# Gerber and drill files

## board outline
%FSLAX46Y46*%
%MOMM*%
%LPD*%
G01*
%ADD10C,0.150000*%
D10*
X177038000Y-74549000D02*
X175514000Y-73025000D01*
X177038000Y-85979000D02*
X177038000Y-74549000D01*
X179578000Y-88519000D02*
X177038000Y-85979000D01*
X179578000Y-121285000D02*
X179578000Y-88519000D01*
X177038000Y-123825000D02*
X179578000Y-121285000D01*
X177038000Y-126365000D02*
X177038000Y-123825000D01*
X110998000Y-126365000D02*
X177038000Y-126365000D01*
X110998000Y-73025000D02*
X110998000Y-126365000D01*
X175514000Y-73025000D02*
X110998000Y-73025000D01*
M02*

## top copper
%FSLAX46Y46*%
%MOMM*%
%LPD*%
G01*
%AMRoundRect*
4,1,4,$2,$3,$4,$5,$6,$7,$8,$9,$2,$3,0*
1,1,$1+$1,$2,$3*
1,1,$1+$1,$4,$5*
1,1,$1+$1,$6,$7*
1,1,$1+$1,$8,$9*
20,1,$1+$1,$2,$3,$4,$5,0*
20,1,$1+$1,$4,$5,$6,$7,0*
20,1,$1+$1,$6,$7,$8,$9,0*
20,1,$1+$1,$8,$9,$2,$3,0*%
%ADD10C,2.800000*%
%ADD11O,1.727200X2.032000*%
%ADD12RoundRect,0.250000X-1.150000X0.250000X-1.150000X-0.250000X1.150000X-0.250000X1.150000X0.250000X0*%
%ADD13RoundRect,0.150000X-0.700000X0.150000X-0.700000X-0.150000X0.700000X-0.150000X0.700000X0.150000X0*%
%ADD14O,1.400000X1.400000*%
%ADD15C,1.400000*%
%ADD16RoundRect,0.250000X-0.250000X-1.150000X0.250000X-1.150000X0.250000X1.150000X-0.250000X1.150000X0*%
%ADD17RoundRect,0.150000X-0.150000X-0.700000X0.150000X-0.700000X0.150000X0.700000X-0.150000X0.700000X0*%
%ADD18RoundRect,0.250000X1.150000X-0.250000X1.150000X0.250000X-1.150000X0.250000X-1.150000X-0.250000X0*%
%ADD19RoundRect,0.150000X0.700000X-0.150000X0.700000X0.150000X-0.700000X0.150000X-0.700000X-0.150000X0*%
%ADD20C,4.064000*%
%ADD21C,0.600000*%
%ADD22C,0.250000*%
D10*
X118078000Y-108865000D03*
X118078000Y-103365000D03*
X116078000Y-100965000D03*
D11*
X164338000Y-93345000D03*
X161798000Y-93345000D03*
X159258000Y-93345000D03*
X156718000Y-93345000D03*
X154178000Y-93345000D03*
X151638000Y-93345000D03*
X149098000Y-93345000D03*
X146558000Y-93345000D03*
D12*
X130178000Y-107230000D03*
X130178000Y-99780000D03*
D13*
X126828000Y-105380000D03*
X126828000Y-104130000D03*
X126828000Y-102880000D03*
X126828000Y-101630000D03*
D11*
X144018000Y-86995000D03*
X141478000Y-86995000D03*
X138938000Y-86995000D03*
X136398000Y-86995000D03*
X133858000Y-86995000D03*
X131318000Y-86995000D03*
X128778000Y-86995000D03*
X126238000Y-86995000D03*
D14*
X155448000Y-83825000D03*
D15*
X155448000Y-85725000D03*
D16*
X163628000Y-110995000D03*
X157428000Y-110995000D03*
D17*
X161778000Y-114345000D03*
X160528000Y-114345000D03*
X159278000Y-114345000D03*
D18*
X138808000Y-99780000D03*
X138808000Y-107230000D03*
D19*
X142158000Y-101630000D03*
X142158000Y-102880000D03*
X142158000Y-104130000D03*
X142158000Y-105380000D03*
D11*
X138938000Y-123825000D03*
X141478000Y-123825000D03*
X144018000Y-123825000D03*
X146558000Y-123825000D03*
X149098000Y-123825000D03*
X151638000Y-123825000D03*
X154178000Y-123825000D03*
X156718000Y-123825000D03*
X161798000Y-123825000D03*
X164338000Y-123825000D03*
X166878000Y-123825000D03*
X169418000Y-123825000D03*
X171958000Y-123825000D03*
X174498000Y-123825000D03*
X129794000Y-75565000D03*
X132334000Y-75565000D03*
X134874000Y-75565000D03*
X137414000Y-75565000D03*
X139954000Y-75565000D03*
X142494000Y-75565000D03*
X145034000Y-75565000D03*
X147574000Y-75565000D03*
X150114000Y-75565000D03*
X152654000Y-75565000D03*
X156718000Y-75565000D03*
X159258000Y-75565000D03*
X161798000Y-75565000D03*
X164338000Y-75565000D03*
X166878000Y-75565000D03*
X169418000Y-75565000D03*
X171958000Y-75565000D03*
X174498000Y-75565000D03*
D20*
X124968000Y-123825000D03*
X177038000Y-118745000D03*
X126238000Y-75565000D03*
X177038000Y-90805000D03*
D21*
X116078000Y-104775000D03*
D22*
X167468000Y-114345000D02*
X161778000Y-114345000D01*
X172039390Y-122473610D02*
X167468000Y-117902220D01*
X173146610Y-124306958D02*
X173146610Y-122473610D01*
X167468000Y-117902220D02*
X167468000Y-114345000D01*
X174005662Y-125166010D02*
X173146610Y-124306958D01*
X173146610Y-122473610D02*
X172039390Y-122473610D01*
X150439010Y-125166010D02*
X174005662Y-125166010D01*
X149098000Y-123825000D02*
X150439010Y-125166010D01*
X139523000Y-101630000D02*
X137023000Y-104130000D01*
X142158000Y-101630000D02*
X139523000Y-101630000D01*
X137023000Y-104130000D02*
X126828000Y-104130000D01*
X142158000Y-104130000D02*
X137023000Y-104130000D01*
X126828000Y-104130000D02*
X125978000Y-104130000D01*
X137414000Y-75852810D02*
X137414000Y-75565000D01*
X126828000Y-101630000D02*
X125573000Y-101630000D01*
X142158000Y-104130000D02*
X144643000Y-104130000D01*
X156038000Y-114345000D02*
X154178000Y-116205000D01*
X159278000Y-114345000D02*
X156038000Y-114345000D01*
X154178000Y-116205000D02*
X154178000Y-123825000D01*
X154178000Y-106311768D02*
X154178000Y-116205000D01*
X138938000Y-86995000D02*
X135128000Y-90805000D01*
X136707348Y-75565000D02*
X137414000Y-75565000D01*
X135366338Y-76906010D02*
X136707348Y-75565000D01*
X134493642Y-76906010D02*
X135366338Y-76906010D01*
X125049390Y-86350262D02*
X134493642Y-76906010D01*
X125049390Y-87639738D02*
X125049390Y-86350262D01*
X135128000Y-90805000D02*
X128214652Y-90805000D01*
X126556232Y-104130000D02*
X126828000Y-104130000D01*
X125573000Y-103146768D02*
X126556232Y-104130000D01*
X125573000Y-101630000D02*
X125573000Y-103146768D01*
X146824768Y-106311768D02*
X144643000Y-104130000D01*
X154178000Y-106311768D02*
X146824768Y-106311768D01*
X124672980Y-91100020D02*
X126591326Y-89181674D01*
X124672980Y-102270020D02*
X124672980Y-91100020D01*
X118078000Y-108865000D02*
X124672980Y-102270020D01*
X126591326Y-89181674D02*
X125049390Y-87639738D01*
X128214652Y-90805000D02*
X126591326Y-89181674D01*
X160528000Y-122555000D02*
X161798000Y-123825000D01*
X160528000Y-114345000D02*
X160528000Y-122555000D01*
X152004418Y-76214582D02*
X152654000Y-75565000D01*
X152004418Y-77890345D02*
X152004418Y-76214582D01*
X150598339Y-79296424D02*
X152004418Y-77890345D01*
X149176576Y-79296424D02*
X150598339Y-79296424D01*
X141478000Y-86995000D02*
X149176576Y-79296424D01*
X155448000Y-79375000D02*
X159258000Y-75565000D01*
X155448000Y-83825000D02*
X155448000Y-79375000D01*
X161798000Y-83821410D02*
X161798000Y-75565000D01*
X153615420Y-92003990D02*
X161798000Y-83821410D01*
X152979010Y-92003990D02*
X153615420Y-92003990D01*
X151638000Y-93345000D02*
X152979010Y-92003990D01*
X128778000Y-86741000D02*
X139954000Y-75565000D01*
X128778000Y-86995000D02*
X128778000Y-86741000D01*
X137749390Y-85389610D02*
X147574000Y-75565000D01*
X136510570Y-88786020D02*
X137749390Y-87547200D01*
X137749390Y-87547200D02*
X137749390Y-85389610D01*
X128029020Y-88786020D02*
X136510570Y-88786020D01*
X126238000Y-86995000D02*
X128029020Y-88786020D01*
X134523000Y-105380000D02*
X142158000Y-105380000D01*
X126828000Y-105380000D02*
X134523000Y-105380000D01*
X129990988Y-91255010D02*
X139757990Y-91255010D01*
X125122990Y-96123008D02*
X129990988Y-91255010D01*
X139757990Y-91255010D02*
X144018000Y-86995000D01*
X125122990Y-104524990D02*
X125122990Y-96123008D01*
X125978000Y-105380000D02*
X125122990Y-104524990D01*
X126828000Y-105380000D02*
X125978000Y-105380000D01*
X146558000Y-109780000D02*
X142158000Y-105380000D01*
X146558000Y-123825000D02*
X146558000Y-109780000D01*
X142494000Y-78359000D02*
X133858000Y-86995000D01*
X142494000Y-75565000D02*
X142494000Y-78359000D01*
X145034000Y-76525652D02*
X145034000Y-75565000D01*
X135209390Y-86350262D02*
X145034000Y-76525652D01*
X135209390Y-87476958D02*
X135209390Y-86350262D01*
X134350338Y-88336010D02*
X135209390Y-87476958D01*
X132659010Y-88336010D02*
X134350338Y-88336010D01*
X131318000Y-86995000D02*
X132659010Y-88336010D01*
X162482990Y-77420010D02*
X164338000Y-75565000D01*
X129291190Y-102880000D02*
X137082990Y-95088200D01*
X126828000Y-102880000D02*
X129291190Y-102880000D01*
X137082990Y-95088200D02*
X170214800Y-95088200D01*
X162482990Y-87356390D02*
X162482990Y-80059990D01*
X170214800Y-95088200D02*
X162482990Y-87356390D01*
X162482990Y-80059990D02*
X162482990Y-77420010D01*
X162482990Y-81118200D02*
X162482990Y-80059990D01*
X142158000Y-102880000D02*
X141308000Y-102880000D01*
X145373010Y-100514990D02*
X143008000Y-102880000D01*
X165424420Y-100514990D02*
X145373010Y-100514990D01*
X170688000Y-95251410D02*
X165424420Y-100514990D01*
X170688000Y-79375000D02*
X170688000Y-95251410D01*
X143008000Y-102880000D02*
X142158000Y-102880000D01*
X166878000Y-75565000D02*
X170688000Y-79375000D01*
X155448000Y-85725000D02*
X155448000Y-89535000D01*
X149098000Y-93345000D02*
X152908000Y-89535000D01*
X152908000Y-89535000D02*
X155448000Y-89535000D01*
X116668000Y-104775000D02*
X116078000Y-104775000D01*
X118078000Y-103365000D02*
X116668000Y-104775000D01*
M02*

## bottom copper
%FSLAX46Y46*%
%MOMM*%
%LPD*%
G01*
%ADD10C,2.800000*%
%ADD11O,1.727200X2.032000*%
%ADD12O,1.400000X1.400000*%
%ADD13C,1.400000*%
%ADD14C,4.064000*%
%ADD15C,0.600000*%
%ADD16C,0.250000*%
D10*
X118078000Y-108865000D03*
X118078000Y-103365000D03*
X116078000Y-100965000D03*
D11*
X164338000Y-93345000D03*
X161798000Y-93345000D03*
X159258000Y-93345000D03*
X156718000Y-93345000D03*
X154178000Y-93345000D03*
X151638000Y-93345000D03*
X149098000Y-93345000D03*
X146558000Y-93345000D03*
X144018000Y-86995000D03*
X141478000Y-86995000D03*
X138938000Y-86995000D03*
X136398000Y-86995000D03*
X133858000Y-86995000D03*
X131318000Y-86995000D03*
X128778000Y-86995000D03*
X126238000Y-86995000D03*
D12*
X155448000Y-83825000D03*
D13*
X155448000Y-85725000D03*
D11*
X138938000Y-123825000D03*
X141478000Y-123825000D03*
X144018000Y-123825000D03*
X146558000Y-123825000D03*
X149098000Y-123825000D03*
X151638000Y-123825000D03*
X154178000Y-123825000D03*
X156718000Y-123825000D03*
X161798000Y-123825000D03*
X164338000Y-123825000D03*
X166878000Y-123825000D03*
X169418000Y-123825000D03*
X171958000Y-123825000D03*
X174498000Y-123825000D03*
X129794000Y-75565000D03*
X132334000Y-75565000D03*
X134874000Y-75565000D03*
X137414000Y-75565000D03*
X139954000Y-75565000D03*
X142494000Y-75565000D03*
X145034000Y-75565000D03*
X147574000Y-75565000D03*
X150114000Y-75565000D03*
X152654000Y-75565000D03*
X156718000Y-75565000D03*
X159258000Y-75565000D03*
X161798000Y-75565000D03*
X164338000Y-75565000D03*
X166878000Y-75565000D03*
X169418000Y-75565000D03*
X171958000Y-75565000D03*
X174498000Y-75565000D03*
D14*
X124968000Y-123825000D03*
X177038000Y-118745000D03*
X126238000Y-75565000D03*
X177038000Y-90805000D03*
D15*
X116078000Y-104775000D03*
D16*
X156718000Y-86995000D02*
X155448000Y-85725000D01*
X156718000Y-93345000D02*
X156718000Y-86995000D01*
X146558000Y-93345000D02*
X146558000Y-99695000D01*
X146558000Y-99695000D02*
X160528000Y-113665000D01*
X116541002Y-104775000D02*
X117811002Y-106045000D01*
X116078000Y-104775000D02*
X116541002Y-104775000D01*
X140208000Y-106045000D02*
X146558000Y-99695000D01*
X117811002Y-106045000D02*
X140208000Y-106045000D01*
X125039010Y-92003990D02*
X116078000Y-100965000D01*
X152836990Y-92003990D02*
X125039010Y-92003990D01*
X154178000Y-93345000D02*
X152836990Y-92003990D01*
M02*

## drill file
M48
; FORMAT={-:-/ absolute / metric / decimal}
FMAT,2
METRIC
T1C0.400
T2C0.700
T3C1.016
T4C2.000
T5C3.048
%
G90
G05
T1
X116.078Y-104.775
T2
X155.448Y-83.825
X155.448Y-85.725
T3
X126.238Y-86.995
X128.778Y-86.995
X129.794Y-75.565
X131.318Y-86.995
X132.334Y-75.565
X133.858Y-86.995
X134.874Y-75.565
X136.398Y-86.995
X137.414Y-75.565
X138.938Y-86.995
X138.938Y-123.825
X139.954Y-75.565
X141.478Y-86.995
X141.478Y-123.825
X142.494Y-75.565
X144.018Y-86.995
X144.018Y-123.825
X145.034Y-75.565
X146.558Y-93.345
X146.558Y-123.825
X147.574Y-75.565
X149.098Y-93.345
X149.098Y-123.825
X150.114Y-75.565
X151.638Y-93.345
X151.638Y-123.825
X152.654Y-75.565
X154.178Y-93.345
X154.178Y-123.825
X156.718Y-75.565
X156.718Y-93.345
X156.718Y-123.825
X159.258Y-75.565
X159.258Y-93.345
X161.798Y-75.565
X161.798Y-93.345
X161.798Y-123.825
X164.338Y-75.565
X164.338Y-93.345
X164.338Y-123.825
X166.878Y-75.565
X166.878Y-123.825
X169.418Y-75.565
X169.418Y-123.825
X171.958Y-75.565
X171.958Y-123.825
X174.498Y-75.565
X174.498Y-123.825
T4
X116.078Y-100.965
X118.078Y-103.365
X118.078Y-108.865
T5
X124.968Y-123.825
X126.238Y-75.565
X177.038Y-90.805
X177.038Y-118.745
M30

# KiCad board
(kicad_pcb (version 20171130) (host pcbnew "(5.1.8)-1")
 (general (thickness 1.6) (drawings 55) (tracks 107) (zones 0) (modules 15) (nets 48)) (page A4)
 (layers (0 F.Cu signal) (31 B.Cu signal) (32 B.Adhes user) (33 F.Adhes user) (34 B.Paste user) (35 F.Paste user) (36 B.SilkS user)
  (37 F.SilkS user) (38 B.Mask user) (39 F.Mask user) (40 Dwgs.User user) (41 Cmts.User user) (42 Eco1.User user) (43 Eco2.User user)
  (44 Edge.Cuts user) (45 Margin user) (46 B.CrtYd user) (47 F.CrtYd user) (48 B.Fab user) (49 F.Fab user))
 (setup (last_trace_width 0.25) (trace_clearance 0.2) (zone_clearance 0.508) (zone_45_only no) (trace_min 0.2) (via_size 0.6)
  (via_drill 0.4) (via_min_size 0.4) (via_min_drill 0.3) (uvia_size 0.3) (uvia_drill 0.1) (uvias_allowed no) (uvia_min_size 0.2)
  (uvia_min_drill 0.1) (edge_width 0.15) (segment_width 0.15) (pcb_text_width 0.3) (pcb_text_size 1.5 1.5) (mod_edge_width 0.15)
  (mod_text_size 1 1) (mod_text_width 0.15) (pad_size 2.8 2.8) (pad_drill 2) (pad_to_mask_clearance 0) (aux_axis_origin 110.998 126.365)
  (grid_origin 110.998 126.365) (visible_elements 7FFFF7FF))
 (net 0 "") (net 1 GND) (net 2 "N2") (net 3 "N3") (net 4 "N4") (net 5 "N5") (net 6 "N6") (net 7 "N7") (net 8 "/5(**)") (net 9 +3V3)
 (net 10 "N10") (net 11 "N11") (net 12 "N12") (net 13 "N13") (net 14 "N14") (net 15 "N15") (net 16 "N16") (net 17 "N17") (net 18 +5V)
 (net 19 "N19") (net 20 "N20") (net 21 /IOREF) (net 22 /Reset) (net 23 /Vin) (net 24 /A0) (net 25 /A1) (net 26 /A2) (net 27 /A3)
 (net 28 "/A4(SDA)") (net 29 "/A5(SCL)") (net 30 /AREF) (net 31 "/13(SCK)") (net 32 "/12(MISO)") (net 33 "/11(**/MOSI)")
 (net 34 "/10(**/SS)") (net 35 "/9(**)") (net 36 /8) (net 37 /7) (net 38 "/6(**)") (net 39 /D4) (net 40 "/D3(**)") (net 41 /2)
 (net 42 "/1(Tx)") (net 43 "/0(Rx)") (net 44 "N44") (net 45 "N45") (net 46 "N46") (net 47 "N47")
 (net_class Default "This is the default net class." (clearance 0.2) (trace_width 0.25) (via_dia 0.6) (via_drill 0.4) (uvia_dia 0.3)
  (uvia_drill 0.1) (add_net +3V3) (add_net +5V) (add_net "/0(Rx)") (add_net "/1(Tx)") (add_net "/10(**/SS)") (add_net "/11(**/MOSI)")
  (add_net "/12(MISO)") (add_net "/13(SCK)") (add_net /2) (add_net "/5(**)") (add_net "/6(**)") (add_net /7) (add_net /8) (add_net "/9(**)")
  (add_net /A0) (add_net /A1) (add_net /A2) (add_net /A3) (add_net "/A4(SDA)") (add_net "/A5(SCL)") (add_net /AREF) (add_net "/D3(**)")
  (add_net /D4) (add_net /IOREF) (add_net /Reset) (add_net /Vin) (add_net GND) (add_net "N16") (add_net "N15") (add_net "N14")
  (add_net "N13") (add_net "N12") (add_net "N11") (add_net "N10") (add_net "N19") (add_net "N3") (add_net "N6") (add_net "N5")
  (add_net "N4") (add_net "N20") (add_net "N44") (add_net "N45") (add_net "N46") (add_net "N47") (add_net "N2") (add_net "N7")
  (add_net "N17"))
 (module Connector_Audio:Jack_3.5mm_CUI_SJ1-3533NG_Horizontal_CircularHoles (layer F.Cu) (at 116.078 100.965)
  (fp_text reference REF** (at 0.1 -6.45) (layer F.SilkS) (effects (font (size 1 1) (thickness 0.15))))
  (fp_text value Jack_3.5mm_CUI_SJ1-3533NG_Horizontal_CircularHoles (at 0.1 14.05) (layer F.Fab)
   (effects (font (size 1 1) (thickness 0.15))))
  (pad R thru_hole circle (at 2 7.9) (size 2.8 2.8) (drill 2) (layers *.Cu *.Mask) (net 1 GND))
  (pad T thru_hole circle (at 2 2.4) (size 2.8 2.8) (drill 2) (layers *.Cu *.Mask) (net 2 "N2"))
  (pad S thru_hole circle (at 0 0) (size 2.8 2.8) (drill 2) (layers *.Cu *.Mask) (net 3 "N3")))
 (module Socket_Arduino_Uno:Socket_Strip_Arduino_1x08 (layer F.Cu) (at 146.558 93.345)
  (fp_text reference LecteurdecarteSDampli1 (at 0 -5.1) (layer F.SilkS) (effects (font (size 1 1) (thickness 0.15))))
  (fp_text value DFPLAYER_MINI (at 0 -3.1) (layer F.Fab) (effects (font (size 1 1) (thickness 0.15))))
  (pad 8 thru_hole oval (at 17.78 0) (size 1.7272 2.032) (drill 1.016) (layers *.Cu *.Mask F.SilkS) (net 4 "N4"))
  (pad 7 thru_hole oval (at 15.24 0) (size 1.7272 2.032) (drill 1.016) (layers *.Cu *.Mask F.SilkS) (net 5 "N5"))
  (pad 6 thru_hole oval (at 12.7 0) (size 1.7272 2.032) (drill 1.016) (layers *.Cu *.Mask F.SilkS) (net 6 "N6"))
  (pad 5 thru_hole oval (at 10.16 0) (size 1.7272 2.032) (drill 1.016) (layers *.Cu *.Mask F.SilkS) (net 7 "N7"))
  (pad 4 thru_hole oval (at 7.62 0) (size 1.7272 2.032) (drill 1.016) (layers *.Cu *.Mask F.SilkS) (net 3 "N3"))
  (pad 3 thru_hole oval (at 5.08 0) (size 1.7272 2.032) (drill 1.016) (layers *.Cu *.Mask F.SilkS) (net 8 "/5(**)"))
  (pad 2 thru_hole oval (at 2.54 0) (size 1.7272 2.032) (drill 1.016) (layers *.Cu *.Mask F.SilkS) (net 7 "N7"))
  (pad 1 thru_hole oval (at 0 0) (size 1.7272 2.032) (drill 1.016) (layers *.Cu *.Mask F.SilkS) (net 2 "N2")))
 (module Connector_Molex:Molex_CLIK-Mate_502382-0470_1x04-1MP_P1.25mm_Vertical (layer F.Cu) (at 128.778 103.505 270)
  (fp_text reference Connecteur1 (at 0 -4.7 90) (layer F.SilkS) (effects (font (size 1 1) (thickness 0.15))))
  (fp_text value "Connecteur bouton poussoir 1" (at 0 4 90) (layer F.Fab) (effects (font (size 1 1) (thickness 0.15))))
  (pad MP smd roundrect (at 3.725 -1.4 270) (size 1 2.8) (layers F.Cu F.Paste F.Mask) (roundrect_rratio 0.25))
  (pad MP smd roundrect (at -3.725 -1.4 270) (size 1 2.8) (layers F.Cu F.Paste F.Mask) (roundrect_rratio 0.25))
  (pad 4 smd roundrect (at 1.875 1.95 270) (size 0.6 1.7) (layers F.Cu F.Paste F.Mask) (roundrect_rratio 0.25) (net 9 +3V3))
  (pad 3 smd roundrect (at 0.625 1.95 270) (size 0.6 1.7) (layers F.Cu F.Paste F.Mask) (roundrect_rratio 0.25) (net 1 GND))
  (pad 2 smd roundrect (at -0.625 1.95 270) (size 0.6 1.7) (layers F.Cu F.Paste F.Mask) (roundrect_rratio 0.25) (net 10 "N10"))
  (pad 1 smd roundrect (at -1.875 1.95 270) (size 0.6 1.7) (layers F.Cu F.Paste F.Mask) (roundrect_rratio 0.25) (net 1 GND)))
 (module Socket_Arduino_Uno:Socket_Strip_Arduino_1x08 (layer F.Cu) (at 126.238 86.995)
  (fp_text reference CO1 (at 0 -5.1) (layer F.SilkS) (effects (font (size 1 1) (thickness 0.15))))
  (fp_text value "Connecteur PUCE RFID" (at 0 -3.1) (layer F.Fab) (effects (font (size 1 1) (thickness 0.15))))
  (pad 8 thru_hole oval (at 17.78 0) (size 1.7272 2.032) (drill 1.016) (layers *.Cu *.Mask F.SilkS) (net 9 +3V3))
  (pad 7 thru_hole oval (at 15.24 0) (size 1.7272 2.032) (drill 1.016) (layers *.Cu *.Mask F.SilkS) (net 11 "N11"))
  (pad 6 thru_hole oval (at 12.7 0) (size 1.7272 2.032) (drill 1.016) (layers *.Cu *.Mask F.SilkS) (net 1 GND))
  (pad 5 thru_hole oval (at 10.16 0) (size 1.7272 2.032) (drill 1.016) (layers *.Cu *.Mask F.SilkS) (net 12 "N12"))
  (pad 4 thru_hole oval (at 7.62 0) (size 1.7272 2.032) (drill 1.016) (layers *.Cu *.Mask F.SilkS) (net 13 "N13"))
  (pad 3 thru_hole oval (at 5.08 0) (size 1.7272 2.032) (drill 1.016) (layers *.Cu *.Mask F.SilkS) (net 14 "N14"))
  (pad 2 thru_hole oval (at 2.54 0) (size 1.7272 2.032) (drill 1.016) (layers *.Cu *.Mask F.SilkS) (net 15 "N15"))
  (pad 1 thru_hole oval (at 0 0) (size 1.7272 2.032) (drill 1.016) (layers *.Cu *.Mask F.SilkS) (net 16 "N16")))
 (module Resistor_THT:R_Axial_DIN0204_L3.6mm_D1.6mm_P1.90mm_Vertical (layer F.Cu) (at 155.448 85.725 90)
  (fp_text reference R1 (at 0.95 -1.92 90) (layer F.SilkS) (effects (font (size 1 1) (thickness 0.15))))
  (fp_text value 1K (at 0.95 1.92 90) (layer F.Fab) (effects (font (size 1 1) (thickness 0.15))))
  (pad 2 thru_hole oval (at 1.9 0 90) (size 1.4 1.4) (drill 0.7) (layers *.Cu *.Mask) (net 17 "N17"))
  (pad 1 thru_hole circle (at 0 0 90) (size 1.4 1.4) (drill 0.7) (layers *.Cu *.Mask) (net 7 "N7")))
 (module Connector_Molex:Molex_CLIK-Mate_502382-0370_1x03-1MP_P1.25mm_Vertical (layer F.Cu) (at 160.528 112.395)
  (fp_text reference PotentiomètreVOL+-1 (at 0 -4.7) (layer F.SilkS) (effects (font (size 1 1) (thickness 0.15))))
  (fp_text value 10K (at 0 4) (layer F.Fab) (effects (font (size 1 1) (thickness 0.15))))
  (pad MP smd roundrect (at 3.1 -1.4) (size 1 2.8) (layers F.Cu F.Paste F.Mask) (roundrect_rratio 0.25))
  (pad MP smd roundrect (at -3.1 -1.4) (size 1 2.8) (layers F.Cu F.Paste F.Mask) (roundrect_rratio 0.25))
  (pad 3 smd roundrect (at 1.25 1.95) (size 0.6 1.7) (layers F.Cu F.Paste F.Mask) (roundrect_rratio 0.25) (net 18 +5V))
  (pad 2 smd roundrect (at 0 1.95) (size 0.6 1.7) (layers F.Cu F.Paste F.Mask) (roundrect_rratio 0.25) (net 2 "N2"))
  (pad 1 smd roundrect (at -1.25 1.95) (size 0.6 1.7) (layers F.Cu F.Paste F.Mask) (roundrect_rratio 0.25) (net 1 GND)))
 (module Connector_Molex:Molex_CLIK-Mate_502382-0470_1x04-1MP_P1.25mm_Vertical (layer F.Cu) (at 140.208 103.505 90)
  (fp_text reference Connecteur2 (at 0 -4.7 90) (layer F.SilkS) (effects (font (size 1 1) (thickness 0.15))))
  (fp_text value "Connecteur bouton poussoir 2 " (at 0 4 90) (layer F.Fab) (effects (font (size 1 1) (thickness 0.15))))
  (pad MP smd roundrect (at 3.725 -1.4 90) (size 1 2.8) (layers F.Cu F.Paste F.Mask) (roundrect_rratio 0.25))
  (pad MP smd roundrect (at -3.725 -1.4 90) (size 1 2.8) (layers F.Cu F.Paste F.Mask) (roundrect_rratio 0.25))
  (pad 1 smd roundrect (at 1.875 1.95 90) (size 0.6 1.7) (layers F.Cu F.Paste F.Mask) (roundrect_rratio 0.25) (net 1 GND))
  (pad 2 smd roundrect (at 0.625 1.95 90) (size 0.6 1.7) (layers F.Cu F.Paste F.Mask) (roundrect_rratio 0.25) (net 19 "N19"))
  (pad 3 smd roundrect (at -0.625 1.95 90) (size 0.6 1.7) (layers F.Cu F.Paste F.Mask) (roundrect_rratio 0.25) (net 1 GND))
  (pad 4 smd roundrect (at -1.875 1.95 90) (size 0.6 1.7) (layers F.Cu F.Paste F.Mask) (roundrect_rratio 0.25) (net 9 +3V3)))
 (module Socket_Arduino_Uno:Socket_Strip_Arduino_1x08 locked (layer F.Cu) (at 138.938 123.825)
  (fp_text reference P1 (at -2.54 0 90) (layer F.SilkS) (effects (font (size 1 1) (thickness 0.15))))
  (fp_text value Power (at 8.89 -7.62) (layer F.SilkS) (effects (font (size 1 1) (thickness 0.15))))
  (pad 1 thru_hole oval (at 0 0) (size 1.7272 2.032) (drill 1.016) (layers *.Cu *.Mask F.SilkS) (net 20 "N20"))
  (pad 2 thru_hole oval (at 2.54 0) (size 1.7272 2.032) (drill 1.016) (layers *.Cu *.Mask F.SilkS) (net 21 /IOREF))
  (pad 3 thru_hole oval (at 5.08 0) (size 1.7272 2.032) (drill 1.016) (layers *.Cu *.Mask F.SilkS) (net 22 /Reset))
  (pad 4 thru_hole oval (at 7.62 0) (size 1.7272 2.032) (drill 1.016) (layers *.Cu *.Mask F.SilkS) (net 9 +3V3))
  (pad 5 thru_hole oval (at 10.16 0) (size 1.7272 2.032) (drill 1.016) (layers *.Cu *.Mask F.SilkS) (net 18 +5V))
  (pad 6 thru_hole oval (at 12.7 0) (size 1.7272 2.032) (drill 1.016) (layers *.Cu *.Mask F.SilkS) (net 1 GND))
  (pad 7 thru_hole oval (at 15.24 0) (size 1.7272 2.032) (drill 1.016) (layers *.Cu *.Mask F.SilkS) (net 1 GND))
  (pad 8 thru_hole oval (at 17.78 0) (size 1.7272 2.032) (drill 1.016) (layers *.Cu *.Mask F.SilkS) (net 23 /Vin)))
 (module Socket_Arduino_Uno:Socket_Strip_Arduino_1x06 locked (layer F.Cu) (at 161.798 123.825)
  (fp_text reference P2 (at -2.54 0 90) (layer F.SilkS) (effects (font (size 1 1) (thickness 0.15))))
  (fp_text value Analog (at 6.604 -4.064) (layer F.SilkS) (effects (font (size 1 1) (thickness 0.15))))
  (pad 1 thru_hole oval (at 0 0) (size 1.7272 2.032) (drill 1.016) (layers *.Cu *.Mask F.SilkS) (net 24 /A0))
  (pad 2 thru_hole oval (at 2.54 0) (size 1.7272 2.032) (drill 1.016) (layers *.Cu *.Mask F.SilkS) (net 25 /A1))
  (pad 3 thru_hole oval (at 5.08 0) (size 1.7272 2.032) (drill 1.016) (layers *.Cu *.Mask F.SilkS) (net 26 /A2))
  (pad 4 thru_hole oval (at 7.62 0) (size 1.7272 2.032) (drill 1.016) (layers *.Cu *.Mask F.SilkS) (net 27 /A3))
  (pad 5 thru_hole oval (at 10.16 0) (size 1.7272 2.032) (drill 1.016) (layers *.Cu *.Mask F.SilkS) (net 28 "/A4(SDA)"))
  (pad 6 thru_hole oval (at 12.7 0) (size 1.7272 2.032) (drill 1.016) (layers *.Cu *.Mask F.SilkS) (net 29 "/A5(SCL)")))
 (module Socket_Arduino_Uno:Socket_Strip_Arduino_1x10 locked (layer F.Cu) (at 129.794 75.565)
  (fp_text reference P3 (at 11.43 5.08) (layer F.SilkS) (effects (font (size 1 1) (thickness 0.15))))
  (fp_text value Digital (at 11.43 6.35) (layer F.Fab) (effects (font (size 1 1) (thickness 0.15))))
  (pad 1 thru_hole oval (at 0 0) (size 1.7272 2.032) (drill 1.016) (layers *.Cu *.Mask F.SilkS) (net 29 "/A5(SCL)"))
  (pad 2 thru_hole oval (at 2.54 0) (size 1.7272 2.032) (drill 1.016) (layers *.Cu *.Mask F.SilkS) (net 28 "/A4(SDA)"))
  (pad 3 thru_hole oval (at 5.08 0) (size 1.7272 2.032) (drill 1.016) (layers *.Cu *.Mask F.SilkS) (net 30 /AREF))
  (pad 4 thru_hole oval (at 7.62 0) (size 1.7272 2.032) (drill 1.016) (layers *.Cu *.Mask F.SilkS) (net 1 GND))
  (pad 5 thru_hole oval (at 10.16 0) (size 1.7272 2.032) (drill 1.016) (layers *.Cu *.Mask F.SilkS) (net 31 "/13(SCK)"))
  (pad 6 thru_hole oval (at 12.7 0) (size 1.7272 2.032) (drill 1.016) (layers *.Cu *.Mask F.SilkS) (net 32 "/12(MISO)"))
  (pad 7 thru_hole oval (at 15.24 0) (size 1.7272 2.032) (drill 1.016) (layers *.Cu *.Mask F.SilkS) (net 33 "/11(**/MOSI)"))
  (pad 8 thru_hole oval (at 17.78 0) (size 1.7272 2.032) (drill 1.016) (layers *.Cu *.Mask F.SilkS) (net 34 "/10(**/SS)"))
  (pad 9 thru_hole oval (at 20.32 0) (size 1.7272 2.032) (drill 1.016) (layers *.Cu *.Mask F.SilkS) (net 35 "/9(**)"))
  (pad 10 thru_hole oval (at 22.86 0) (size 1.7272 2.032) (drill 1.016) (layers *.Cu *.Mask F.SilkS) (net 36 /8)))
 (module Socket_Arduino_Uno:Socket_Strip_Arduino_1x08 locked (layer F.Cu) (at 156.718 75.565)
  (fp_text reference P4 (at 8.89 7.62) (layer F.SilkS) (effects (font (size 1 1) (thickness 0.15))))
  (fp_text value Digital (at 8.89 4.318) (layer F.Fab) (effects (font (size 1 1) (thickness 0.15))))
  (pad 1 thru_hole oval (at 0 0) (size 1.7272 2.032) (drill 1.016) (layers *.Cu *.Mask F.SilkS) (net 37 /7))
  (pad 2 thru_hole oval (at 2.54 0) (size 1.7272 2.032) (drill 1.016) (layers *.Cu *.Mask F.SilkS) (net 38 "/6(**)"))
  (pad 3 thru_hole oval (at 5.08 0) (size 1.7272 2.032) (drill 1.016) (layers *.Cu *.Mask F.SilkS) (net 8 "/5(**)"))
  (pad 4 thru_hole oval (at 7.62 0) (size 1.7272 2.032) (drill 1.016) (layers *.Cu *.Mask F.SilkS) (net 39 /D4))
  (pad 5 thru_hole oval (at 10.16 0) (size 1.7272 2.032) (drill 1.016) (layers *.Cu *.Mask F.SilkS) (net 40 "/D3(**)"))
  (pad 6 thru_hole oval (at 12.7 0) (size 1.7272 2.032) (drill 1.016) (layers *.Cu *.Mask F.SilkS) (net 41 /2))
  (pad 7 thru_hole oval (at 15.24 0) (size 1.7272 2.032) (drill 1.016) (layers *.Cu *.Mask F.SilkS) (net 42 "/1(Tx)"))
  (pad 8 thru_hole oval (at 17.78 0) (size 1.7272 2.032) (drill 1.016) (layers *.Cu *.Mask F.SilkS) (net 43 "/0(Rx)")))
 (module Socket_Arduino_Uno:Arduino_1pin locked (layer F.Cu) (at 124.968 123.825)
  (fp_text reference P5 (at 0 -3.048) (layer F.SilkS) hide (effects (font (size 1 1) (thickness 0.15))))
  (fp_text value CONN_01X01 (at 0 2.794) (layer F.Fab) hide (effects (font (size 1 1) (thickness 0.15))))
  (pad 1 thru_hole circle (at 0 0) (size 4.064 4.064) (drill 3.048) (layers *.Cu *.Mask F.SilkS) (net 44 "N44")))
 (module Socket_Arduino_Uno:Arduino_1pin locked (layer F.Cu) (at 177.038 118.745)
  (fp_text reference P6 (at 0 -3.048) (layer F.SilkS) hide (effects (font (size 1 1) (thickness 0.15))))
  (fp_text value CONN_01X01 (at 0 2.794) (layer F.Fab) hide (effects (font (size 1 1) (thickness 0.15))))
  (pad 1 thru_hole circle (at 0 0) (size 4.064 4.064) (drill 3.048) (layers *.Cu *.Mask F.SilkS) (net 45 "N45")))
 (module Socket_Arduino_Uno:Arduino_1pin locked (layer F.Cu) (at 126.238 75.565)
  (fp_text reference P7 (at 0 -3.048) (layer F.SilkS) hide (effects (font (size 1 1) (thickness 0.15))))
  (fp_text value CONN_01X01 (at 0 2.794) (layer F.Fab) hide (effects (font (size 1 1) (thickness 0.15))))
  (pad 1 thru_hole circle (at 0 0) (size 4.064 4.064) (drill 3.048) (layers *.Cu *.Mask F.SilkS) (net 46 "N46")))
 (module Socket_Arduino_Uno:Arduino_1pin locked (layer F.Cu) (at 177.038 90.805)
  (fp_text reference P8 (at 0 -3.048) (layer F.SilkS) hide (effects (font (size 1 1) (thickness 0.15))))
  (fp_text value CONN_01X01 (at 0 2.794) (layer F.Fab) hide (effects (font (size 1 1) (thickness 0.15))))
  (pad 1 thru_hole circle (at 0 0) (size 4.064 4.064) (drill 3.048) (layers *.Cu *.Mask F.SilkS) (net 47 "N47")))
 (gr_line (start 177.038 74.549) (end 175.514 73.025) (angle 90) (layer Edge.Cuts) (width 0.15))
 (gr_line (start 177.038 85.979) (end 177.038 74.549) (angle 90) (layer Edge.Cuts) (width 0.15))
 (gr_line (start 179.578 88.519) (end 177.038 85.979) (angle 90) (layer Edge.Cuts) (width 0.15))
 (gr_line (start 179.578 121.285) (end 179.578 88.519) (angle 90) (layer Edge.Cuts) (width 0.15))
 (gr_line (start 177.038 123.825) (end 179.578 121.285) (angle 90) (layer Edge.Cuts) (width 0.15))
 (gr_line (start 177.038 126.365) (end 177.038 123.825) (angle 90) (layer Edge.Cuts) (width 0.15))
 (gr_line (start 110.998 126.365) (end 177.038 126.365) (angle 90) (layer Edge.Cuts) (width 0.15))
 (gr_line (start 110.998 73.025) (end 110.998 126.365) (angle 90) (layer Edge.Cuts) (width 0.15))
 (gr_line (start 175.514 73.025) (end 110.998 73.025) (angle 90) (layer Edge.Cuts) (width 0.15))
 (segment (start 167.468 114.345) (end 161.778 114.345) (width 0.25) (layer F.Cu) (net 18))
 (segment (start 172.03939 122.47361) (end 167.468 117.90222) (width 0.25) (layer F.Cu) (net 18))
 (segment (start 173.14661 124.306958) (end 173.14661 122.47361) (width 0.25) (layer F.Cu) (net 18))
 (segment (start 167.468 117.90222) (end 167.468 114.345) (width 0.25) (layer F.Cu) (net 18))
 (segment (start 174.005662 125.16601) (end 173.14661 124.306958) (width 0.25) (layer F.Cu) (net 18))
 (segment (start 173.14661 122.47361) (end 172.03939 122.47361) (width 0.25) (layer F.Cu) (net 18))
 (segment (start 150.43901 125.16601) (end 174.005662 125.16601) (width 0.25) (layer F.Cu) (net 18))
 (segment (start 149.098 123.825) (end 150.43901 125.16601) (width 0.25) (layer F.Cu) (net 18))
 (segment (start 139.523 101.63) (end 137.023 104.13) (width 0.25) (layer F.Cu) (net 1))
 (segment (start 142.158 101.63) (end 139.523 101.63) (width 0.25) (layer F.Cu) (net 1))
 (segment (start 137.023 104.13) (end 126.828 104.13) (width 0.25) (layer F.Cu) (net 1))
 (segment (start 142.158 104.13) (end 137.023 104.13) (width 0.25) (layer F.Cu) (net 1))
 (segment (start 126.828 104.13) (end 125.978 104.13) (width 0.25) (layer F.Cu) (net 1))
 (segment (start 137.414 75.85281) (end 137.414 75.565) (width 0.25) (layer F.Cu) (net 1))
 (segment (start 126.828 101.63) (end 125.573 101.63) (width 0.25) (layer F.Cu) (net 1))
 (segment (start 142.158 104.13) (end 144.643 104.13) (width 0.25) (layer F.Cu) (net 1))
 (segment (start 156.038 114.345) (end 154.178 116.205) (width 0.25) (layer F.Cu) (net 1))
 (segment (start 159.278 114.345) (end 156.038 114.345) (width 0.25) (layer F.Cu) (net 1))
 (segment (start 154.178 116.205) (end 154.178 123.825) (width 0.25) (layer F.Cu) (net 1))
 (segment (start 154.178 106.311768) (end 154.178 116.205) (width 0.25) (layer F.Cu) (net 1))
 (segment (start 138.938 86.995) (end 135.128 90.805) (width 0.25) (layer F.Cu) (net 1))
 (segment (start 136.707348 75.565) (end 137.414 75.565) (width 0.25) (layer F.Cu) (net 1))
 (segment (start 135.366338 76.90601) (end 136.707348 75.565) (width 0.25) (layer F.Cu) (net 1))
 (segment (start 134.493642 76.90601) (end 135.366338 76.90601) (width 0.25) (layer F.Cu) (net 1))
 (segment (start 125.04939 86.350262) (end 134.493642 76.90601) (width 0.25) (layer F.Cu) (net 1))
 (segment (start 125.04939 87.639738) (end 125.04939 86.350262) (width 0.25) (layer F.Cu) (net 1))
 (segment (start 135.128 90.805) (end 128.214652 90.805) (width 0.25) (layer F.Cu) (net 1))
 (segment (start 126.556232 104.13) (end 126.828 104.13) (width 0.25) (layer F.Cu) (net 1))
 (segment (start 125.573 103.146768) (end 126.556232 104.13) (width 0.25) (layer F.Cu) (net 1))
 (segment (start 125.573 101.63) (end 125.573 103.146768) (width 0.25) (layer F.Cu) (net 1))
 (segment (start 146.824768 106.311768) (end 144.643 104.13) (width 0.25) (layer F.Cu) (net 1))
 (segment (start 154.178 106.311768) (end 146.824768 106.311768) (width 0.25) (layer F.Cu) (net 1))
 (segment (start 124.67298 91.10002) (end 126.591326 89.181674) (width 0.25) (layer F.Cu) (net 1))
 (segment (start 124.67298 102.27002) (end 124.67298 91.10002) (width 0.25) (layer F.Cu) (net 1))
 (segment (start 118.078 108.865) (end 124.67298 102.27002) (width 0.25) (layer F.Cu) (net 1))
 (segment (start 126.591326 89.181674) (end 125.04939 87.639738) (width 0.25) (layer F.Cu) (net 1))
 (segment (start 128.214652 90.805) (end 126.591326 89.181674) (width 0.25) (layer F.Cu) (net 1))
 (segment (start 160.528 122.555) (end 161.798 123.825) (width 0.25) (layer F.Cu) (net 24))
 (segment (start 160.528 114.345) (end 160.528 122.555) (width 0.25) (layer F.Cu) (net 24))
 (segment (start 152.004418 76.214582) (end 152.654 75.565) (width 0.25) (layer F.Cu) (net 36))
 (segment (start 152.004418 77.890345) (end 152.004418 76.214582) (width 0.25) (layer F.Cu) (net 36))
 (segment (start 150.598339 79.296424) (end 152.004418 77.890345) (width 0.25) (layer F.Cu) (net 36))
 (segment (start 149.176576 79.296424) (end 150.598339 79.296424) (width 0.25) (layer F.Cu) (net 36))
 (segment (start 141.478 86.995) (end 149.176576 79.296424) (width 0.25) (layer F.Cu) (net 36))
 (segment (start 155.448 79.375) (end 159.258 75.565) (width 0.25) (layer F.Cu) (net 38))
 (segment (start 155.448 83.825) (end 155.448 79.375) (width 0.25) (layer F.Cu) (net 38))
 (segment (start 161.798 83.82141) (end 161.798 75.565) (width 0.25) (layer F.Cu) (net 8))
 (segment (start 153.61542 92.00399) (end 161.798 83.82141) (width 0.25) (layer F.Cu) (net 8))
 (segment (start 152.97901 92.00399) (end 153.61542 92.00399) (width 0.25) (layer F.Cu) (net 8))
 (segment (start 151.638 93.345) (end 152.97901 92.00399) (width 0.25) (layer F.Cu) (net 8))
 (segment (start 128.778 86.741) (end 139.954 75.565) (width 0.25) (layer F.Cu) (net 31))
 (segment (start 128.778 86.995) (end 128.778 86.741) (width 0.25) (layer F.Cu) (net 31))
 (segment (start 137.74939 85.38961) (end 147.574 75.565) (width 0.25) (layer F.Cu) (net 34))
 (segment (start 136.51057 88.78602) (end 137.74939 87.5472) (width 0.25) (layer F.Cu) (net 34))
 (segment (start 137.74939 87.5472) (end 137.74939 85.38961) (width 0.25) (layer F.Cu) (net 34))
 (segment (start 128.02902 88.78602) (end 136.51057 88.78602) (width 0.25) (layer F.Cu) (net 34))
 (segment (start 126.238 86.995) (end 128.02902 88.78602) (width 0.25) (layer F.Cu) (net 34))
 (segment (start 134.523 105.38) (end 142.158 105.38) (width 0.25) (layer F.Cu) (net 9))
 (segment (start 126.828 105.38) (end 134.523 105.38) (width 0.25) (layer F.Cu) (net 9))
 (segment (start 129.990988 91.25501) (end 139.75799 91.25501) (width 0.25) (layer F.Cu) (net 9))
 (segment (start 125.12299 96.123008) (end 129.990988 91.25501) (width 0.25) (layer F.Cu) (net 9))
 (segment (start 139.75799 91.25501) (end 144.018 86.995) (width 0.25) (layer F.Cu) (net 9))
 (segment (start 125.12299 104.52499) (end 125.12299 96.123008) (width 0.25) (layer F.Cu) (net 9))
 (segment (start 125.978 105.38) (end 125.12299 104.52499) (width 0.25) (layer F.Cu) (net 9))
 (segment (start 126.828 105.38) (end 125.978 105.38) (width 0.25) (layer F.Cu) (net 9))
 (segment (start 146.558 109.78) (end 142.158 105.38) (width 0.25) (layer F.Cu) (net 9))
 (segment (start 146.558 123.825) (end 146.558 109.78) (width 0.25) (layer F.Cu) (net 9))
 (segment (start 142.494 78.359) (end 133.858 86.995) (width 0.25) (layer F.Cu) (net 32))
 (segment (start 142.494 75.565) (end 142.494 78.359) (width 0.25) (layer F.Cu) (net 32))
 (segment (start 145.034 76.525652) (end 145.034 75.565) (width 0.25) (layer F.Cu) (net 33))
 (segment (start 135.20939 86.350262) (end 145.034 76.525652) (width 0.25) (layer F.Cu) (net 33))
 (segment (start 135.20939 87.476958) (end 135.20939 86.350262) (width 0.25) (layer F.Cu) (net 33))
 (segment (start 134.350338 88.33601) (end 135.20939 87.476958) (width 0.25) (layer F.Cu) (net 33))
 (segment (start 132.65901 88.33601) (end 134.350338 88.33601) (width 0.25) (layer F.Cu) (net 33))
 (segment (start 131.318 86.995) (end 132.65901 88.33601) (width 0.25) (layer F.Cu) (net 33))
 (segment (start 162.48299 77.42001) (end 164.338 75.565) (width 0.25) (layer F.Cu) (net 39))
 (segment (start 129.29119 102.88) (end 137.08299 95.0882) (width 0.25) (layer F.Cu) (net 39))
 (segment (start 126.828 102.88) (end 129.29119 102.88) (width 0.25) (layer F.Cu) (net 39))
 (segment (start 137.08299 95.0882) (end 170.2148 95.0882) (width 0.25) (layer F.Cu) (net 39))
 (segment (start 162.48299 87.35639) (end 162.48299 80.05999) (width 0.25) (layer F.Cu) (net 39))
 (segment (start 170.2148 95.0882) (end 162.48299 87.35639) (width 0.25) (layer F.Cu) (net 39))
 (segment (start 162.48299 80.05999) (end 162.48299 77.42001) (width 0.25) (layer F.Cu) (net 39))
 (segment (start 162.48299 81.1182) (end 162.48299 80.05999) (width 0.25) (layer F.Cu) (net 39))
 (segment (start 142.158 102.88) (end 141.308 102.88) (width 0.25) (layer F.Cu) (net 40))
 (segment (start 145.37301 100.51499) (end 143.008 102.88) (width 0.25) (layer F.Cu) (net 40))
 (segment (start 165.42442 100.51499) (end 145.37301 100.51499) (width 0.25) (layer F.Cu) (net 40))
 (segment (start 170.688 95.25141) (end 165.42442 100.51499) (width 0.25) (layer F.Cu) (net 40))
 (segment (start 170.688 79.375) (end 170.688 95.25141) (width 0.25) (layer F.Cu) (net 40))
 (segment (start 143.008 102.88) (end 142.158 102.88) (width 0.25) (layer F.Cu) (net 40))
 (segment (start 166.878 75.565) (end 170.688 79.375) (width 0.25) (layer F.Cu) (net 40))
 (segment (start 155.448 85.725) (end 155.448 89.535) (width 0.25) (layer F.Cu) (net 7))
 (segment (start 149.098 93.345) (end 152.908 89.535) (width 0.25) (layer F.Cu) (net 7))
 (segment (start 152.908 89.535) (end 155.448 89.535) (width 0.25) (layer F.Cu) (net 7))
 (segment (start 156.718 86.995) (end 155.448 85.725) (width 0.25) (layer B.Cu) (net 7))
 (segment (start 156.718 93.345) (end 156.718 86.995) (width 0.25) (layer B.Cu) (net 7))
 (segment (start 146.558 93.345) (end 146.558 99.695) (width 0.25) (layer B.Cu) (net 2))
 (segment (start 146.558 99.695) (end 160.528 113.665) (width 0.25) (layer B.Cu) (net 2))
 (via (at 116.078 104.775) (size 0.6) (drill 0.4) (layers F.Cu B.Cu) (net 2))
 (segment (start 116.668 104.775) (end 116.078 104.775) (width 0.25) (layer F.Cu) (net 2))
 (segment (start 118.078 103.365) (end 116.668 104.775) (width 0.25) (layer F.Cu) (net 2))
 (segment (start 116.541002 104.775) (end 117.811002 106.045) (width 0.25) (layer B.Cu) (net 2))
 (segment (start 116.078 104.775) (end 116.541002 104.775) (width 0.25) (layer B.Cu) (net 2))
 (segment (start 140.208 106.045) (end 146.558 99.695) (width 0.25) (layer B.Cu) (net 2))
 (segment (start 117.811002 106.045) (end 140.208 106.045) (width 0.25) (layer B.Cu) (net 2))
 (segment (start 125.03901 92.00399) (end 116.078 100.965) (width 0.25) (layer B.Cu) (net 3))
 (segment (start 152.83699 92.00399) (end 125.03901 92.00399) (width 0.25) (layer B.Cu) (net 3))
 (segment (start 154.178 93.345) (end 152.83699 92.00399) (width 0.25) (layer B.Cu) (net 3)))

